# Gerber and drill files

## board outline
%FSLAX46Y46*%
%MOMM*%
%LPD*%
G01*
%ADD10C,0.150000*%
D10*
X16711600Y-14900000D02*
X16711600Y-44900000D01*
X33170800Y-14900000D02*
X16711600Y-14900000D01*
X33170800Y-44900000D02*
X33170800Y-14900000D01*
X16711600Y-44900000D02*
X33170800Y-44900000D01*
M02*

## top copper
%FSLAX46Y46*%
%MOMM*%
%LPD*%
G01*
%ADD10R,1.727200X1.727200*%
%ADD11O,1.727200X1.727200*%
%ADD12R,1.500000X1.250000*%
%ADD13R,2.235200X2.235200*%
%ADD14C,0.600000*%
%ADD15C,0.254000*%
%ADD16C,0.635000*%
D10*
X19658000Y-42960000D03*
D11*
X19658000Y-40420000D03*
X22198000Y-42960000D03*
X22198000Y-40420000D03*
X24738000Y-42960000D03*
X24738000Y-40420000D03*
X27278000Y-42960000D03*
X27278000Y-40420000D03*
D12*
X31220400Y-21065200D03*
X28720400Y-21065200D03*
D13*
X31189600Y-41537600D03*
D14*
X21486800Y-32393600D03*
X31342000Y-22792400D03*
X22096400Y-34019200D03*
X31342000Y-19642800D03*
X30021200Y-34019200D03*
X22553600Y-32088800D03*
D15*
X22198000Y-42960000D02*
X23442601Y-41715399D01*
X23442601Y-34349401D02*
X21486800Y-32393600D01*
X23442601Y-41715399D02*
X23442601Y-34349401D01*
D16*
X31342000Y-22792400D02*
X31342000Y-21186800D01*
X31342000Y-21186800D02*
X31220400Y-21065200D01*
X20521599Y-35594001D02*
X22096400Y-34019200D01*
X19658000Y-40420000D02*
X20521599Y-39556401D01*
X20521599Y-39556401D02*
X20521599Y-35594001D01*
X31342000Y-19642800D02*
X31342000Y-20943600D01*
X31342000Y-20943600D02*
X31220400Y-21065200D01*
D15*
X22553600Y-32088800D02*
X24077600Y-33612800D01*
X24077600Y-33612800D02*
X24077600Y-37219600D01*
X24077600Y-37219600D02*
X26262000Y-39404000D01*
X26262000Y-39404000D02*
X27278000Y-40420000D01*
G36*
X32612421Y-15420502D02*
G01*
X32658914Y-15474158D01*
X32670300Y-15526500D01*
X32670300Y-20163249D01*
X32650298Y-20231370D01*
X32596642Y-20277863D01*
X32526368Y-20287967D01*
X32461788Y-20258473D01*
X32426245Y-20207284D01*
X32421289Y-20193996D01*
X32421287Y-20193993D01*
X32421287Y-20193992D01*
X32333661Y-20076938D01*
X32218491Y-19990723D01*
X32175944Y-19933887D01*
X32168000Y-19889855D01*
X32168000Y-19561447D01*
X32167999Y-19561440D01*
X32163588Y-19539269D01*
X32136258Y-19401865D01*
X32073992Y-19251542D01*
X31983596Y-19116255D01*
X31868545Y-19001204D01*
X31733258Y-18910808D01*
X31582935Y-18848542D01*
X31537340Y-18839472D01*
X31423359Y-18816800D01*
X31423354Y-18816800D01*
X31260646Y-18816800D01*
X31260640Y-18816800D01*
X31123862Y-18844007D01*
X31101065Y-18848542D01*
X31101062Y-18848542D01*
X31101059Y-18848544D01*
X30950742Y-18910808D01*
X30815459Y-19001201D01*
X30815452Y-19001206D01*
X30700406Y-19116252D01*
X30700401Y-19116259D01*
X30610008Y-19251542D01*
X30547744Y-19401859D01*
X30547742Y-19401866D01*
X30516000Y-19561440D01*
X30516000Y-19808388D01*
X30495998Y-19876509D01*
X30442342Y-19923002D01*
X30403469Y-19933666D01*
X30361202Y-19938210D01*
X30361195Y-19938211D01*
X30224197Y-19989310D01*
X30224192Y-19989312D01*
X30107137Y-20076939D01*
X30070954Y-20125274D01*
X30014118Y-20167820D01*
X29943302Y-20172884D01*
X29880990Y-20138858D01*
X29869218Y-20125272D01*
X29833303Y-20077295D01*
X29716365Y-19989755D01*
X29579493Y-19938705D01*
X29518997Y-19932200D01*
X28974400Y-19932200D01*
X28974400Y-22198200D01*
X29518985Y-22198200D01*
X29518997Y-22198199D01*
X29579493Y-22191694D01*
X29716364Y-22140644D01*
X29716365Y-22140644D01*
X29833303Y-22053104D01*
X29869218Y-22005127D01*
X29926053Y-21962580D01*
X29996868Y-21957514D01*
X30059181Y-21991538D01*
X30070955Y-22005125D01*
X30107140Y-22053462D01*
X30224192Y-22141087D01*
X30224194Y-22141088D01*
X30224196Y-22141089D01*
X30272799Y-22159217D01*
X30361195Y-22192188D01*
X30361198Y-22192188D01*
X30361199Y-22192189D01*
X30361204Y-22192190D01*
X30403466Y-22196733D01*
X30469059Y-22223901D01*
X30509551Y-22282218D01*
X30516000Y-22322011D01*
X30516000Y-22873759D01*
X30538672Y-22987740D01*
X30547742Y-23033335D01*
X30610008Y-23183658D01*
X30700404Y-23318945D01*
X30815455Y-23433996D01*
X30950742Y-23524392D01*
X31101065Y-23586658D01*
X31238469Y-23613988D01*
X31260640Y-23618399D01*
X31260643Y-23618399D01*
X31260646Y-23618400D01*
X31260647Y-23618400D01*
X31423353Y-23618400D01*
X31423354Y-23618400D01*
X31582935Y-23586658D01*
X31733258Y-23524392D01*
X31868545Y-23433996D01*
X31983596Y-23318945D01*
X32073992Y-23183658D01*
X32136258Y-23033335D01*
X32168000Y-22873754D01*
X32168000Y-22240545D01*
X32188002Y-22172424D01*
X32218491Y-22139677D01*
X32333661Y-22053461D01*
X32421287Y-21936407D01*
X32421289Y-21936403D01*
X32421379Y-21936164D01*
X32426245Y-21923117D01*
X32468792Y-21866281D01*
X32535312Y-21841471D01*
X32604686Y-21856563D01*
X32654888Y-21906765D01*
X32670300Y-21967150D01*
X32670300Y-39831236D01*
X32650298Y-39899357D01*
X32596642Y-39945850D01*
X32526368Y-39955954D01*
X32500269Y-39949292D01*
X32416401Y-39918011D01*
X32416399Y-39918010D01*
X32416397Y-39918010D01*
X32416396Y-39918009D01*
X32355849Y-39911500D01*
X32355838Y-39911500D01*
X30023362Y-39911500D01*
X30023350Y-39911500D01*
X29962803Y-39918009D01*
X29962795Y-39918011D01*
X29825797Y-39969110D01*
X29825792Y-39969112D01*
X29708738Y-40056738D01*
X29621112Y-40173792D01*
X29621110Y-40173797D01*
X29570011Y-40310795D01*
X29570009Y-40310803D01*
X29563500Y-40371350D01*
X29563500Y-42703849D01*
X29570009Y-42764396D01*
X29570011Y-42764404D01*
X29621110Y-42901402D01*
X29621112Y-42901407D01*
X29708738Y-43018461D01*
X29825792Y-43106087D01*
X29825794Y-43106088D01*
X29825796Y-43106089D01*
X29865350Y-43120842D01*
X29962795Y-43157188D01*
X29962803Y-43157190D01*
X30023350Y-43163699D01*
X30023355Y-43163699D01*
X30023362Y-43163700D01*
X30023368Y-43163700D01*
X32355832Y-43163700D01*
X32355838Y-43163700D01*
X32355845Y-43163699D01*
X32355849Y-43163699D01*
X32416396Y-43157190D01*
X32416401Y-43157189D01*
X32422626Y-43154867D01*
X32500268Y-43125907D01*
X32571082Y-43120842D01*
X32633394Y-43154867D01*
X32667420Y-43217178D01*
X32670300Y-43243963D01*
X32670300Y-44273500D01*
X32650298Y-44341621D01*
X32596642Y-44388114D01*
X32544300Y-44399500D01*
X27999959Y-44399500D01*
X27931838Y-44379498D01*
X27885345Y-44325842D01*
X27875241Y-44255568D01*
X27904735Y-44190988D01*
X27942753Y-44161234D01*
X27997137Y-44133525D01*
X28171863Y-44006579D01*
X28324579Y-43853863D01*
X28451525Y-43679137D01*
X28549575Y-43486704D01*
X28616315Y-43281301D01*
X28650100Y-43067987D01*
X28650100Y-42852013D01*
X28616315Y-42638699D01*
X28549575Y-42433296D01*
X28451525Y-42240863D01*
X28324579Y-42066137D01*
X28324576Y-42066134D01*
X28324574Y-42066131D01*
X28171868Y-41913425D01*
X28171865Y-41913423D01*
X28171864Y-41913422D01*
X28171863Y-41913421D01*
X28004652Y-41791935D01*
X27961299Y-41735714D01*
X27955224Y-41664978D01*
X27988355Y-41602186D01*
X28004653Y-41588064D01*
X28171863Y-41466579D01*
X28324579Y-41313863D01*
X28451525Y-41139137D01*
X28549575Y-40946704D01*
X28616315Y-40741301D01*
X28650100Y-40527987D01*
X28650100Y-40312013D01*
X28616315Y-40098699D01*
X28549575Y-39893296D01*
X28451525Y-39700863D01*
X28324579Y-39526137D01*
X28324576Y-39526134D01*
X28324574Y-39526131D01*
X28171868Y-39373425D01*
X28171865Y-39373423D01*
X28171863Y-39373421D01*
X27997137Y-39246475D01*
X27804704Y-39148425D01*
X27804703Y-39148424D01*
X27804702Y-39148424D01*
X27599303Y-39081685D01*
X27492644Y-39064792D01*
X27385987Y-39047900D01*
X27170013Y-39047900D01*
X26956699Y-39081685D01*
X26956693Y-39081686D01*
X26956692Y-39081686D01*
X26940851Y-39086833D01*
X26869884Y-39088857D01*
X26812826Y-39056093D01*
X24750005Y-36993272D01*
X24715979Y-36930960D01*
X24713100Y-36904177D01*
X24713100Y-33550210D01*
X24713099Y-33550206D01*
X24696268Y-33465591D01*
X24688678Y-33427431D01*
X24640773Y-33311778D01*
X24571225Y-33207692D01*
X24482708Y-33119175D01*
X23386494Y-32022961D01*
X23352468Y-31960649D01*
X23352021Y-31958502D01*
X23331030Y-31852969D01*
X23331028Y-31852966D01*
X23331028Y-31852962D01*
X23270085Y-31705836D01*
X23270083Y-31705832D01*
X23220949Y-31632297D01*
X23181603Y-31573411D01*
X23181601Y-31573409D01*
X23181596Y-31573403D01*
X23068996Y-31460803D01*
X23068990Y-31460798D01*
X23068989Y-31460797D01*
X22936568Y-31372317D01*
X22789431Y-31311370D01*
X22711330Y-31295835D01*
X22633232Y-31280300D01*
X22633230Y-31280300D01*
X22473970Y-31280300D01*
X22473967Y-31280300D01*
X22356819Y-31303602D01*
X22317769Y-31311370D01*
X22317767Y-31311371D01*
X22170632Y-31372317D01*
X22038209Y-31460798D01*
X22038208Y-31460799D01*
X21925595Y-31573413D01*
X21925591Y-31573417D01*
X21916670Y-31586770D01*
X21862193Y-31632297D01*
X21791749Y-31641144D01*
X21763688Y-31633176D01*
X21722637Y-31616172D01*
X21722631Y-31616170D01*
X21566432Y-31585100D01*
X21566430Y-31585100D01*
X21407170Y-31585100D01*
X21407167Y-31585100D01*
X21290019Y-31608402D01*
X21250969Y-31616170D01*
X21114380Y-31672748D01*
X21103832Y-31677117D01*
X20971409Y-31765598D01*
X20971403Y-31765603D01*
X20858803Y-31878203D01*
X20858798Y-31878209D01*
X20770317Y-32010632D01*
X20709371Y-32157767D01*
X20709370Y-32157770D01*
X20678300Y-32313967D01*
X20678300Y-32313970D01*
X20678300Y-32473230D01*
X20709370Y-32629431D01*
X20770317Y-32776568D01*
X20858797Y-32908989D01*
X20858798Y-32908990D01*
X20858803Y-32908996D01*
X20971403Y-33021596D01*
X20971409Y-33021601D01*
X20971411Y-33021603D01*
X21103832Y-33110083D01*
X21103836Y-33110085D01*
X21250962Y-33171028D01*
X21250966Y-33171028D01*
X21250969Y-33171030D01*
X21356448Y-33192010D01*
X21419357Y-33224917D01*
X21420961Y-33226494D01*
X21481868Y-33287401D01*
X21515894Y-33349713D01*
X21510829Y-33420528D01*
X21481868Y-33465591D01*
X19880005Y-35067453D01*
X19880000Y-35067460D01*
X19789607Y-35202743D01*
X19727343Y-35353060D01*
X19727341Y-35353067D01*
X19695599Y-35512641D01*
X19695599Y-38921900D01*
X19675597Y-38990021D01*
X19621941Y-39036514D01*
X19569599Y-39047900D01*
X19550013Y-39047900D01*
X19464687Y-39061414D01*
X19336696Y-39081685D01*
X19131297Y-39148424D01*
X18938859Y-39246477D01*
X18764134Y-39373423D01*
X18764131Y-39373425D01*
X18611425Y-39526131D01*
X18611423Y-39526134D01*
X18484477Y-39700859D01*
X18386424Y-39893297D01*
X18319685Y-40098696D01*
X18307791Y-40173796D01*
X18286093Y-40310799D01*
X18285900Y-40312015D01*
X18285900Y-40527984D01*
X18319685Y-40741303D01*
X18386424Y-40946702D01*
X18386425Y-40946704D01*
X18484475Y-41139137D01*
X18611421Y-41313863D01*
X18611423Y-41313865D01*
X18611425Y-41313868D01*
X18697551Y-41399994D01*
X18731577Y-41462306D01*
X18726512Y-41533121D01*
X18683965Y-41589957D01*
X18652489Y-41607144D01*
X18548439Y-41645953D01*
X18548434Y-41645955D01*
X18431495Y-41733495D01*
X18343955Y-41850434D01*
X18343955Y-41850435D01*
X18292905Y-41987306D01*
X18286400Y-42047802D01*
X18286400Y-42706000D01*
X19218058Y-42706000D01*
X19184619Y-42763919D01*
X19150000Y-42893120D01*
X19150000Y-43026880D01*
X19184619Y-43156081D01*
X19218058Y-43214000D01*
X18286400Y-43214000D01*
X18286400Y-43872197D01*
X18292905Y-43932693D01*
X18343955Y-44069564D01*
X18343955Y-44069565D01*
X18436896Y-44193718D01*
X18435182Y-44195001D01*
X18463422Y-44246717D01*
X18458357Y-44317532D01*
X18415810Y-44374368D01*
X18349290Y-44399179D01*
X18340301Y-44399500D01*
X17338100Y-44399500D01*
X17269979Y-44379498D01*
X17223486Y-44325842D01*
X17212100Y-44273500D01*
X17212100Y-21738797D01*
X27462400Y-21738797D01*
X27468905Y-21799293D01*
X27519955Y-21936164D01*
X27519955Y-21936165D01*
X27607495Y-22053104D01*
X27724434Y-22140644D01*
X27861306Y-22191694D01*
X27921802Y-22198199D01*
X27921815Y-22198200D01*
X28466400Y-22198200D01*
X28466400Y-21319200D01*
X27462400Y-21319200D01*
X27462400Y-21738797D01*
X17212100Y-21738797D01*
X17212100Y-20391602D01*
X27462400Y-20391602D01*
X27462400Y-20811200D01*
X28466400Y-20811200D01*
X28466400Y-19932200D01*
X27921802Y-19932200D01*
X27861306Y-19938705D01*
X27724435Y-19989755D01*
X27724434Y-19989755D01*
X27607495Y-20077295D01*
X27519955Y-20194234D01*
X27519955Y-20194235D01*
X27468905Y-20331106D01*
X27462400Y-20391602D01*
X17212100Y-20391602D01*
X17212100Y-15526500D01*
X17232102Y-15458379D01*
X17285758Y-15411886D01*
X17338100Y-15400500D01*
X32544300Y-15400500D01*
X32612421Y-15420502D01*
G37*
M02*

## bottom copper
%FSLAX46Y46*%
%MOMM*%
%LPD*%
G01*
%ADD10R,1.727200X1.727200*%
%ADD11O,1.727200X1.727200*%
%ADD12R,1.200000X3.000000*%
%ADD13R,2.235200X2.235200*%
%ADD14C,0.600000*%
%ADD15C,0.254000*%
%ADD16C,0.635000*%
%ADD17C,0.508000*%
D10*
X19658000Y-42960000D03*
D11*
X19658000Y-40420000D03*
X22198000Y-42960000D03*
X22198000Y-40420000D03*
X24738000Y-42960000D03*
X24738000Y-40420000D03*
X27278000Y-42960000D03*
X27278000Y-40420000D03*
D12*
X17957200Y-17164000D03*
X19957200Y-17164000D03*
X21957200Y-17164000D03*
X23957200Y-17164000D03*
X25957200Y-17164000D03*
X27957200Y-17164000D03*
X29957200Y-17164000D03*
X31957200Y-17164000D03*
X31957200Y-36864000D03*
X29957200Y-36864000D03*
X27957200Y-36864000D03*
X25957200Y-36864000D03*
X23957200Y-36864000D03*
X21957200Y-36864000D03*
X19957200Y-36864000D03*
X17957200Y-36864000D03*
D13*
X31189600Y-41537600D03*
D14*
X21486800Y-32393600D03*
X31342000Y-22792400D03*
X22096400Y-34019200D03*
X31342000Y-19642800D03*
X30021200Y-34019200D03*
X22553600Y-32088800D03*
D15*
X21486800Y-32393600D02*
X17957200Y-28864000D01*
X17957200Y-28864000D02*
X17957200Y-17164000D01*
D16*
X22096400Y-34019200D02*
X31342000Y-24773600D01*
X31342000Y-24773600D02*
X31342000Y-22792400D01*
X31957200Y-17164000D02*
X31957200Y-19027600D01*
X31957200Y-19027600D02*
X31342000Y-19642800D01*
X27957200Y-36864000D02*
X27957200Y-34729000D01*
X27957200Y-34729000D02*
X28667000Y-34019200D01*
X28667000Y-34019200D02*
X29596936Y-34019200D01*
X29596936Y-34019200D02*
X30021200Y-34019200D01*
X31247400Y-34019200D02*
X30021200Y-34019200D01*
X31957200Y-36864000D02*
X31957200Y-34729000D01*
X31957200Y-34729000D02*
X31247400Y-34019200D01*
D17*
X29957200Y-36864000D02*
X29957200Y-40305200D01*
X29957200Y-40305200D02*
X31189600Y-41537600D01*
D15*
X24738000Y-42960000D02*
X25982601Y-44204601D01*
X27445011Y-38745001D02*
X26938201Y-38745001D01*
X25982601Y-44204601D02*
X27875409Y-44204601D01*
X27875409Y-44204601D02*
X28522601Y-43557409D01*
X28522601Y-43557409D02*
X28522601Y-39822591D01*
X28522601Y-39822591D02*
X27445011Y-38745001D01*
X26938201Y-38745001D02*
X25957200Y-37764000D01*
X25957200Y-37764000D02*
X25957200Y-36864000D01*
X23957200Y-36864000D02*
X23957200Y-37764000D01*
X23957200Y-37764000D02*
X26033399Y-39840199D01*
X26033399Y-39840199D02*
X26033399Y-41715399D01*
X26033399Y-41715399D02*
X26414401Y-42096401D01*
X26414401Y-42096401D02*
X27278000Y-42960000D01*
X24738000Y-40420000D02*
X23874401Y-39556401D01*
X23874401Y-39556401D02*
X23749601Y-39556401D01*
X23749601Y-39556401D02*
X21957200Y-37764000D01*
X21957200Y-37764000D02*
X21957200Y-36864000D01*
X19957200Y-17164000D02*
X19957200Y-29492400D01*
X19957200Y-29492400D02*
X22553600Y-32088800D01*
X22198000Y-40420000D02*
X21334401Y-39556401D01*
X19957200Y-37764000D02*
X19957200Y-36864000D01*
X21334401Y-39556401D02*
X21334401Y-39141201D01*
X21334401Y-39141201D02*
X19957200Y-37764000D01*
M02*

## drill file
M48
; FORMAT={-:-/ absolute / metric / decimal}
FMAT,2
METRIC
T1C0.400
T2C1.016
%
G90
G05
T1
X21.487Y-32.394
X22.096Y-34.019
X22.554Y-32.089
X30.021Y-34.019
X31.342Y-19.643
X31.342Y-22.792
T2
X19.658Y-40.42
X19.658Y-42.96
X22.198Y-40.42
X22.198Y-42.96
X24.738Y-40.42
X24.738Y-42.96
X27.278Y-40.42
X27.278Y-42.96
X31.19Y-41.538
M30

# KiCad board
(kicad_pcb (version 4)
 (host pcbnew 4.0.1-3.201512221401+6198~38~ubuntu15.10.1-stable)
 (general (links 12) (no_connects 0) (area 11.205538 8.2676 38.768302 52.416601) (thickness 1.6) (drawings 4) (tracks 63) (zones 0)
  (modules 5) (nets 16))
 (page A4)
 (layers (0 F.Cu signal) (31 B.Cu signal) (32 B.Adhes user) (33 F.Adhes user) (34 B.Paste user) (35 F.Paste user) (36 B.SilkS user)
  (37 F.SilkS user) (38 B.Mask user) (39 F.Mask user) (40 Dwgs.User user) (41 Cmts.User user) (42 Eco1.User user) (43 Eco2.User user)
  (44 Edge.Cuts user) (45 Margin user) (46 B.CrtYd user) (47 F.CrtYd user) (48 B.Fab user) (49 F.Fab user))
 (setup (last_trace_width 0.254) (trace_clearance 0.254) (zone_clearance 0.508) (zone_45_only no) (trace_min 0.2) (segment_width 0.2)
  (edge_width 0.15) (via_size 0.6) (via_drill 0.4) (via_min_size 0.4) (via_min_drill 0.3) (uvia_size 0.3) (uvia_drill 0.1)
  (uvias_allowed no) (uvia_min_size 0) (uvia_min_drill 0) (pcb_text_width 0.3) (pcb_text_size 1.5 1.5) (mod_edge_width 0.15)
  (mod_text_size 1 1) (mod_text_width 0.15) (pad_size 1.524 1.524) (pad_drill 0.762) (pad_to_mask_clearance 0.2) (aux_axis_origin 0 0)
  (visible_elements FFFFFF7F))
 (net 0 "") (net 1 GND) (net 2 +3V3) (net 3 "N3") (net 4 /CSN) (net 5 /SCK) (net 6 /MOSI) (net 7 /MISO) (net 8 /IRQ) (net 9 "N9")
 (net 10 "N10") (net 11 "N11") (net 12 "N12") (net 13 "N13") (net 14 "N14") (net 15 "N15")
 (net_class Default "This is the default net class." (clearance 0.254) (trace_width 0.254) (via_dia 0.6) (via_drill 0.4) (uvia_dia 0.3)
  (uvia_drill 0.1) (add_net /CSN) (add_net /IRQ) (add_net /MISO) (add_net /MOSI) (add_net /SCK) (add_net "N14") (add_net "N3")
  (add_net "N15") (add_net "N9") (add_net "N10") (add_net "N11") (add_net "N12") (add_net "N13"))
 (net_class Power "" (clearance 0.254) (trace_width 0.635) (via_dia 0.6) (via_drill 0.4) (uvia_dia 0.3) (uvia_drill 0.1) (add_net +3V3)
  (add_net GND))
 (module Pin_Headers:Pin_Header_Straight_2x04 (layer F.Cu) (at 19.658 42.96 90)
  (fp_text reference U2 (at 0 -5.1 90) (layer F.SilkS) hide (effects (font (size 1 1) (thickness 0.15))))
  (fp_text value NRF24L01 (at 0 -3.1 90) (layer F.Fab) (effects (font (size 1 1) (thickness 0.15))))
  (pad 1 thru_hole rect (at 0 0 90) (size 1.7272 1.7272) (drill 1.016) (layers *.Cu *.Mask F.SilkS) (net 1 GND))
  (pad 2 thru_hole oval (at 2.54 0 90) (size 1.7272 1.7272) (drill 1.016) (layers *.Cu *.Mask F.SilkS) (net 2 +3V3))
  (pad 3 thru_hole oval (at 0 2.54 90) (size 1.7272 1.7272) (drill 1.016) (layers *.Cu *.Mask F.SilkS) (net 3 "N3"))
  (pad 4 thru_hole oval (at 2.54 2.54 90) (size 1.7272 1.7272) (drill 1.016) (layers *.Cu *.Mask F.SilkS) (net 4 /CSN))
  (pad 5 thru_hole oval (at 0 5.08 90) (size 1.7272 1.7272) (drill 1.016) (layers *.Cu *.Mask F.SilkS) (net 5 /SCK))
  (pad 6 thru_hole oval (at 2.54 5.08 90) (size 1.7272 1.7272) (drill 1.016) (layers *.Cu *.Mask F.SilkS) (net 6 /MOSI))
  (pad 7 thru_hole oval (at 0 7.62 90) (size 1.7272 1.7272) (drill 1.016) (layers *.Cu *.Mask F.SilkS) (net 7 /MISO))
  (pad 8 thru_hole oval (at 2.54 7.62 90) (size 1.7272 1.7272) (drill 1.016) (layers *.Cu *.Mask F.SilkS) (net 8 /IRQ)))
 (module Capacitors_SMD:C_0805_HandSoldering (layer F.Cu) (at 29.9704 21.0652 180)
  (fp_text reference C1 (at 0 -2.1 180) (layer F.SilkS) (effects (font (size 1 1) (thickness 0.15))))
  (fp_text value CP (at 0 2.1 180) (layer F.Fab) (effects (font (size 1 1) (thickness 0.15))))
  (pad 1 smd rect (at -1.25 0 180) (size 1.5 1.25) (layers F.Cu F.Paste F.Mask) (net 2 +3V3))
  (pad 2 smd rect (at 1.25 0 180) (size 1.5 1.25) (layers F.Cu F.Paste F.Mask) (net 1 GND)))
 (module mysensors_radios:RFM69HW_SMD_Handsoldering (layer B.Cu) (at 17.9572 18.564 270)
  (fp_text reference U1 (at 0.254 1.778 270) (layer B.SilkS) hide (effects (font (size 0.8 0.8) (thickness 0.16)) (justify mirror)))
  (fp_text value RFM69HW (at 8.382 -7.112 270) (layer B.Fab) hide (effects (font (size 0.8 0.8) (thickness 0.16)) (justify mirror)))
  (pad 1 smd rect (at -1.4 0 270) (size 3 1.2) (layers B.Cu B.Paste B.Mask) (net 3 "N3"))
  (pad 2 smd rect (at -1.4 -2 270) (size 3 1.2) (layers B.Cu B.Paste B.Mask) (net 8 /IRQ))
  (pad 3 smd rect (at -1.4 -4 270) (size 3 1.2) (layers B.Cu B.Paste B.Mask) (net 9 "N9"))
  (pad 4 smd rect (at -1.4 -6 270) (size 3 1.2) (layers B.Cu B.Paste B.Mask) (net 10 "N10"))
  (pad 5 smd rect (at -1.4 -8 270) (size 3 1.2) (layers B.Cu B.Paste B.Mask) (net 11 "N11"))
  (pad 6 smd rect (at -1.4 -10 270) (size 3 1.2) (layers B.Cu B.Paste B.Mask) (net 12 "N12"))
  (pad 7 smd rect (at -1.4 -12 270) (size 3 1.2) (layers B.Cu B.Paste B.Mask) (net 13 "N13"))
  (pad 8 smd rect (at -1.4 -14 270) (size 3 1.2) (layers B.Cu B.Paste B.Mask) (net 2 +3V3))
  (pad 9 smd rect (at 18.3 -14 270) (size 3 1.2) (layers B.Cu B.Paste B.Mask) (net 1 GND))
  (pad 10 smd rect (at 18.3 -12 270) (size 3 1.2) (layers B.Cu B.Paste B.Mask) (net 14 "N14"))
  (pad 11 smd rect (at 18.3 -10 270) (size 3 1.2) (layers B.Cu B.Paste B.Mask) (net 1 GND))
  (pad 12 smd rect (at 18.3 -8 270) (size 3 1.2) (layers B.Cu B.Paste B.Mask) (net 5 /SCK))
  (pad 13 smd rect (at 18.3 -6 270) (size 3 1.2) (layers B.Cu B.Paste B.Mask) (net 7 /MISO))
  (pad 14 smd rect (at 18.3 -4 270) (size 3 1.2) (layers B.Cu B.Paste B.Mask) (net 6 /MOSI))
  (pad 15 smd rect (at 18.3 -2 270) (size 3 1.2) (layers B.Cu B.Paste B.Mask) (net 4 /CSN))
  (pad 16 smd rect (at 18.3 0 270) (size 3 1.2) (layers B.Cu B.Paste B.Mask) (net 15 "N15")))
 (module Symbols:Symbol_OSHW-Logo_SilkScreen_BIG (layer F.Cu) (at 24.6872 8.7716)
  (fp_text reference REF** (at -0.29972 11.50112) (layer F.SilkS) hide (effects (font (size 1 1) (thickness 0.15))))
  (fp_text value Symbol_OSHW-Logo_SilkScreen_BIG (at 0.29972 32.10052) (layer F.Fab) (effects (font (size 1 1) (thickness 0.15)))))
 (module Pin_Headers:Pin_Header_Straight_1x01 (layer F.Cu) (at 31.1896 41.5376)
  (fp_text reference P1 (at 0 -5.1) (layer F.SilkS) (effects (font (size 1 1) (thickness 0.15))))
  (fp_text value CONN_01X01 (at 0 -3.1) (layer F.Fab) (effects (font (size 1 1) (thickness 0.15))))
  (pad 1 thru_hole rect (at 0 0) (size 2.2352 2.2352) (drill 1.016) (layers *.Cu *.Mask F.SilkS) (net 14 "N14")))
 (gr_line (start 16.7116 14.9) (end 16.7116 44.9) (layer Edge.Cuts) (width 0.15))
 (gr_line (start 33.1708 14.9) (end 16.7116 14.9) (layer Edge.Cuts) (width 0.15))
 (gr_line (start 33.1708 44.9) (end 33.1708 14.9) (layer Edge.Cuts) (width 0.15))
 (gr_line (start 16.7116 44.9) (end 33.1708 44.9) (layer Edge.Cuts) (width 0.15))
 (segment (start 16.1 14.9) (end 16.1 45.4) (width 0.25) (layer Dwgs.User) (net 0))
 (segment (start 33.6 14.9) (end 16.1 14.9) (width 0.25) (layer Dwgs.User) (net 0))
 (segment (start 33.6 44.9) (end 33.6 14.9) (width 0.25) (layer Dwgs.User) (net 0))
 (segment (start 16.7116 44.9) (end 33.6 44.9) (width 0.25) (layer Dwgs.User) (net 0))
 (segment (start 19.4675 45.5635) (end 31.596 45.5635) (width 0.25) (layer Dwgs.User) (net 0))
 (segment (start 21.4868 32.3936) (end 17.9572 28.864) (width 0.254) (layer B.Cu) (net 3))
 (segment (start 17.9572 28.864) (end 17.9572 17.164) (width 0.254) (layer B.Cu) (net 3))
 (segment (start 22.198 42.96) (end 23.442601 41.715399) (width 0.254) (layer F.Cu) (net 3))
 (segment (start 23.442601 34.349401) (end 21.4868 32.3936) (width 0.254) (layer F.Cu) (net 3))
 (segment (start 23.442601 41.715399) (end 23.442601 34.349401) (width 0.254) (layer F.Cu) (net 3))
 (via (at 21.4868 32.3936) (size 0.6) (drill 0.4) (layers F.Cu B.Cu) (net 3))
 (segment (start 31.342 22.7924) (end 31.342 21.1868) (width 0.635) (layer F.Cu) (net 2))
 (segment (start 31.342 21.1868) (end 31.2204 21.0652) (width 0.635) (layer F.Cu) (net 2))
 (segment (start 22.0964 34.0192) (end 31.342 24.7736) (width 0.635) (layer B.Cu) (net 2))
 (via (at 31.342 22.7924) (size 0.6) (drill 0.4) (layers F.Cu B.Cu) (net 2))
 (segment (start 31.342 24.7736) (end 31.342 22.7924) (width 0.635) (layer B.Cu) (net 2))
 (segment (start 20.521599 35.594001) (end 22.0964 34.0192) (width 0.635) (layer F.Cu) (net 2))
 (via (at 22.0964 34.0192) (size 0.6) (drill 0.4) (layers F.Cu B.Cu) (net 2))
 (segment (start 19.658 40.42) (end 20.521599 39.556401) (width 0.635) (layer F.Cu) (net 2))
 (segment (start 20.521599 39.556401) (end 20.521599 35.594001) (width 0.635) (layer F.Cu) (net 2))
 (segment (start 31.342 19.6428) (end 31.342 20.9436) (width 0.635) (layer F.Cu) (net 2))
 (segment (start 31.342 20.9436) (end 31.2204 21.0652) (width 0.635) (layer F.Cu) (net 2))
 (segment (start 31.9572 17.164) (end 31.9572 19.0276) (width 0.635) (layer B.Cu) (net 2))
 (segment (start 31.9572 19.0276) (end 31.342 19.6428) (width 0.635) (layer B.Cu) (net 2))
 (via (at 31.342 19.6428) (size 0.6) (drill 0.4) (layers F.Cu B.Cu) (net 2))
 (segment (start 27.9572 36.864) (end 27.9572 34.729) (width 0.635) (layer B.Cu) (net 1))
 (segment (start 27.9572 34.729) (end 28.667 34.0192) (width 0.635) (layer B.Cu) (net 1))
 (segment (start 28.667 34.0192) (end 29.596936 34.0192) (width 0.635) (layer B.Cu) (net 1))
 (segment (start 29.596936 34.0192) (end 30.0212 34.0192) (width 0.635) (layer B.Cu) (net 1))
 (segment (start 31.2474 34.0192) (end 30.0212 34.0192) (width 0.635) (layer B.Cu) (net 1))
 (via (at 30.0212 34.0192) (size 0.6) (drill 0.4) (layers F.Cu B.Cu) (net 1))
 (segment (start 31.9572 36.864) (end 31.9572 34.729) (width 0.635) (layer B.Cu) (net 1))
 (segment (start 31.9572 34.729) (end 31.2474 34.0192) (width 0.635) (layer B.Cu) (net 1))
 (segment (start 29.9572 36.864) (end 29.9572 40.3052) (width 0.508) (layer B.Cu) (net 14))
 (segment (start 29.9572 40.3052) (end 31.1896 41.5376) (width 0.508) (layer B.Cu) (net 14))
 (segment (start 24.738 42.96) (end 25.982601 44.204601) (width 0.254) (layer B.Cu) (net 5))
 (segment (start 27.445011 38.745001) (end 26.938201 38.745001) (width 0.254) (layer B.Cu) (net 5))
 (segment (start 25.982601 44.204601) (end 27.875409 44.204601) (width 0.254) (layer B.Cu) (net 5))
 (segment (start 27.875409 44.204601) (end 28.522601 43.557409) (width 0.254) (layer B.Cu) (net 5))
 (segment (start 28.522601 43.557409) (end 28.522601 39.822591) (width 0.254) (layer B.Cu) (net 5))
 (segment (start 28.522601 39.822591) (end 27.445011 38.745001) (width 0.254) (layer B.Cu) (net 5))
 (segment (start 26.938201 38.745001) (end 25.9572 37.764) (width 0.254) (layer B.Cu) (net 5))
 (segment (start 25.9572 37.764) (end 25.9572 36.864) (width 0.254) (layer B.Cu) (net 5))
 (segment (start 23.9572 36.864) (end 23.9572 37.764) (width 0.254) (layer B.Cu) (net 7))
 (segment (start 23.9572 37.764) (end 26.033399 39.840199) (width 0.254) (layer B.Cu) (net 7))
 (segment (start 26.033399 39.840199) (end 26.033399 41.715399) (width 0.254) (layer B.Cu) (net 7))
 (segment (start 26.033399 41.715399) (end 26.414401 42.096401) (width 0.254) (layer B.Cu) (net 7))
 (segment (start 26.414401 42.096401) (end 27.278 42.96) (width 0.254) (layer B.Cu) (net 7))
 (segment (start 24.738 40.42) (end 23.874401 39.556401) (width 0.254) (layer B.Cu) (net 6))
 (segment (start 23.874401 39.556401) (end 23.749601 39.556401) (width 0.254) (layer B.Cu) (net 6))
 (segment (start 23.749601 39.556401) (end 21.9572 37.764) (width 0.254) (layer B.Cu) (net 6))
 (segment (start 21.9572 37.764) (end 21.9572 36.864) (width 0.254) (layer B.Cu) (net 6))
 (segment (start 22.5536 32.0888) (end 24.0776 33.6128) (width 0.254) (layer F.Cu) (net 8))
 (segment (start 24.0776 33.6128) (end 24.0776 37.2196) (width 0.254) (layer F.Cu) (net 8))
 (segment (start 24.0776 37.2196) (end 26.262 39.404) (width 0.254) (layer F.Cu) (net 8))
 (segment (start 26.262 39.404) (end 27.278 40.42) (width 0.254) (layer F.Cu) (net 8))
 (segment (start 19.9572 17.164) (end 19.9572 29.4924) (width 0.254) (layer B.Cu) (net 8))
 (segment (start 19.9572 29.4924) (end 22.5536 32.0888) (width 0.254) (layer B.Cu) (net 8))
 (via (at 22.5536 32.0888) (size 0.6) (drill 0.4) (layers F.Cu B.Cu) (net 8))
 (segment (start 22.198 40.42) (end 21.334401 39.556401) (width 0.254) (layer B.Cu) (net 4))
 (segment (start 19.9572 37.764) (end 19.9572 36.864) (width 0.254) (layer B.Cu) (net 4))
 (segment (start 21.334401 39.556401) (end 21.334401 39.141201) (width 0.254) (layer B.Cu) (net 4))
 (segment (start 21.334401 39.141201) (end 19.9572 37.764) (width 0.254) (layer B.Cu) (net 4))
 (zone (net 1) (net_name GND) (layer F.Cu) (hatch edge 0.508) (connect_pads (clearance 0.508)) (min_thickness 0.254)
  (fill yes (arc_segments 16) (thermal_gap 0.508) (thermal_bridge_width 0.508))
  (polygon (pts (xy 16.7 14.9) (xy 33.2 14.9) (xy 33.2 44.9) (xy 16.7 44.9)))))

